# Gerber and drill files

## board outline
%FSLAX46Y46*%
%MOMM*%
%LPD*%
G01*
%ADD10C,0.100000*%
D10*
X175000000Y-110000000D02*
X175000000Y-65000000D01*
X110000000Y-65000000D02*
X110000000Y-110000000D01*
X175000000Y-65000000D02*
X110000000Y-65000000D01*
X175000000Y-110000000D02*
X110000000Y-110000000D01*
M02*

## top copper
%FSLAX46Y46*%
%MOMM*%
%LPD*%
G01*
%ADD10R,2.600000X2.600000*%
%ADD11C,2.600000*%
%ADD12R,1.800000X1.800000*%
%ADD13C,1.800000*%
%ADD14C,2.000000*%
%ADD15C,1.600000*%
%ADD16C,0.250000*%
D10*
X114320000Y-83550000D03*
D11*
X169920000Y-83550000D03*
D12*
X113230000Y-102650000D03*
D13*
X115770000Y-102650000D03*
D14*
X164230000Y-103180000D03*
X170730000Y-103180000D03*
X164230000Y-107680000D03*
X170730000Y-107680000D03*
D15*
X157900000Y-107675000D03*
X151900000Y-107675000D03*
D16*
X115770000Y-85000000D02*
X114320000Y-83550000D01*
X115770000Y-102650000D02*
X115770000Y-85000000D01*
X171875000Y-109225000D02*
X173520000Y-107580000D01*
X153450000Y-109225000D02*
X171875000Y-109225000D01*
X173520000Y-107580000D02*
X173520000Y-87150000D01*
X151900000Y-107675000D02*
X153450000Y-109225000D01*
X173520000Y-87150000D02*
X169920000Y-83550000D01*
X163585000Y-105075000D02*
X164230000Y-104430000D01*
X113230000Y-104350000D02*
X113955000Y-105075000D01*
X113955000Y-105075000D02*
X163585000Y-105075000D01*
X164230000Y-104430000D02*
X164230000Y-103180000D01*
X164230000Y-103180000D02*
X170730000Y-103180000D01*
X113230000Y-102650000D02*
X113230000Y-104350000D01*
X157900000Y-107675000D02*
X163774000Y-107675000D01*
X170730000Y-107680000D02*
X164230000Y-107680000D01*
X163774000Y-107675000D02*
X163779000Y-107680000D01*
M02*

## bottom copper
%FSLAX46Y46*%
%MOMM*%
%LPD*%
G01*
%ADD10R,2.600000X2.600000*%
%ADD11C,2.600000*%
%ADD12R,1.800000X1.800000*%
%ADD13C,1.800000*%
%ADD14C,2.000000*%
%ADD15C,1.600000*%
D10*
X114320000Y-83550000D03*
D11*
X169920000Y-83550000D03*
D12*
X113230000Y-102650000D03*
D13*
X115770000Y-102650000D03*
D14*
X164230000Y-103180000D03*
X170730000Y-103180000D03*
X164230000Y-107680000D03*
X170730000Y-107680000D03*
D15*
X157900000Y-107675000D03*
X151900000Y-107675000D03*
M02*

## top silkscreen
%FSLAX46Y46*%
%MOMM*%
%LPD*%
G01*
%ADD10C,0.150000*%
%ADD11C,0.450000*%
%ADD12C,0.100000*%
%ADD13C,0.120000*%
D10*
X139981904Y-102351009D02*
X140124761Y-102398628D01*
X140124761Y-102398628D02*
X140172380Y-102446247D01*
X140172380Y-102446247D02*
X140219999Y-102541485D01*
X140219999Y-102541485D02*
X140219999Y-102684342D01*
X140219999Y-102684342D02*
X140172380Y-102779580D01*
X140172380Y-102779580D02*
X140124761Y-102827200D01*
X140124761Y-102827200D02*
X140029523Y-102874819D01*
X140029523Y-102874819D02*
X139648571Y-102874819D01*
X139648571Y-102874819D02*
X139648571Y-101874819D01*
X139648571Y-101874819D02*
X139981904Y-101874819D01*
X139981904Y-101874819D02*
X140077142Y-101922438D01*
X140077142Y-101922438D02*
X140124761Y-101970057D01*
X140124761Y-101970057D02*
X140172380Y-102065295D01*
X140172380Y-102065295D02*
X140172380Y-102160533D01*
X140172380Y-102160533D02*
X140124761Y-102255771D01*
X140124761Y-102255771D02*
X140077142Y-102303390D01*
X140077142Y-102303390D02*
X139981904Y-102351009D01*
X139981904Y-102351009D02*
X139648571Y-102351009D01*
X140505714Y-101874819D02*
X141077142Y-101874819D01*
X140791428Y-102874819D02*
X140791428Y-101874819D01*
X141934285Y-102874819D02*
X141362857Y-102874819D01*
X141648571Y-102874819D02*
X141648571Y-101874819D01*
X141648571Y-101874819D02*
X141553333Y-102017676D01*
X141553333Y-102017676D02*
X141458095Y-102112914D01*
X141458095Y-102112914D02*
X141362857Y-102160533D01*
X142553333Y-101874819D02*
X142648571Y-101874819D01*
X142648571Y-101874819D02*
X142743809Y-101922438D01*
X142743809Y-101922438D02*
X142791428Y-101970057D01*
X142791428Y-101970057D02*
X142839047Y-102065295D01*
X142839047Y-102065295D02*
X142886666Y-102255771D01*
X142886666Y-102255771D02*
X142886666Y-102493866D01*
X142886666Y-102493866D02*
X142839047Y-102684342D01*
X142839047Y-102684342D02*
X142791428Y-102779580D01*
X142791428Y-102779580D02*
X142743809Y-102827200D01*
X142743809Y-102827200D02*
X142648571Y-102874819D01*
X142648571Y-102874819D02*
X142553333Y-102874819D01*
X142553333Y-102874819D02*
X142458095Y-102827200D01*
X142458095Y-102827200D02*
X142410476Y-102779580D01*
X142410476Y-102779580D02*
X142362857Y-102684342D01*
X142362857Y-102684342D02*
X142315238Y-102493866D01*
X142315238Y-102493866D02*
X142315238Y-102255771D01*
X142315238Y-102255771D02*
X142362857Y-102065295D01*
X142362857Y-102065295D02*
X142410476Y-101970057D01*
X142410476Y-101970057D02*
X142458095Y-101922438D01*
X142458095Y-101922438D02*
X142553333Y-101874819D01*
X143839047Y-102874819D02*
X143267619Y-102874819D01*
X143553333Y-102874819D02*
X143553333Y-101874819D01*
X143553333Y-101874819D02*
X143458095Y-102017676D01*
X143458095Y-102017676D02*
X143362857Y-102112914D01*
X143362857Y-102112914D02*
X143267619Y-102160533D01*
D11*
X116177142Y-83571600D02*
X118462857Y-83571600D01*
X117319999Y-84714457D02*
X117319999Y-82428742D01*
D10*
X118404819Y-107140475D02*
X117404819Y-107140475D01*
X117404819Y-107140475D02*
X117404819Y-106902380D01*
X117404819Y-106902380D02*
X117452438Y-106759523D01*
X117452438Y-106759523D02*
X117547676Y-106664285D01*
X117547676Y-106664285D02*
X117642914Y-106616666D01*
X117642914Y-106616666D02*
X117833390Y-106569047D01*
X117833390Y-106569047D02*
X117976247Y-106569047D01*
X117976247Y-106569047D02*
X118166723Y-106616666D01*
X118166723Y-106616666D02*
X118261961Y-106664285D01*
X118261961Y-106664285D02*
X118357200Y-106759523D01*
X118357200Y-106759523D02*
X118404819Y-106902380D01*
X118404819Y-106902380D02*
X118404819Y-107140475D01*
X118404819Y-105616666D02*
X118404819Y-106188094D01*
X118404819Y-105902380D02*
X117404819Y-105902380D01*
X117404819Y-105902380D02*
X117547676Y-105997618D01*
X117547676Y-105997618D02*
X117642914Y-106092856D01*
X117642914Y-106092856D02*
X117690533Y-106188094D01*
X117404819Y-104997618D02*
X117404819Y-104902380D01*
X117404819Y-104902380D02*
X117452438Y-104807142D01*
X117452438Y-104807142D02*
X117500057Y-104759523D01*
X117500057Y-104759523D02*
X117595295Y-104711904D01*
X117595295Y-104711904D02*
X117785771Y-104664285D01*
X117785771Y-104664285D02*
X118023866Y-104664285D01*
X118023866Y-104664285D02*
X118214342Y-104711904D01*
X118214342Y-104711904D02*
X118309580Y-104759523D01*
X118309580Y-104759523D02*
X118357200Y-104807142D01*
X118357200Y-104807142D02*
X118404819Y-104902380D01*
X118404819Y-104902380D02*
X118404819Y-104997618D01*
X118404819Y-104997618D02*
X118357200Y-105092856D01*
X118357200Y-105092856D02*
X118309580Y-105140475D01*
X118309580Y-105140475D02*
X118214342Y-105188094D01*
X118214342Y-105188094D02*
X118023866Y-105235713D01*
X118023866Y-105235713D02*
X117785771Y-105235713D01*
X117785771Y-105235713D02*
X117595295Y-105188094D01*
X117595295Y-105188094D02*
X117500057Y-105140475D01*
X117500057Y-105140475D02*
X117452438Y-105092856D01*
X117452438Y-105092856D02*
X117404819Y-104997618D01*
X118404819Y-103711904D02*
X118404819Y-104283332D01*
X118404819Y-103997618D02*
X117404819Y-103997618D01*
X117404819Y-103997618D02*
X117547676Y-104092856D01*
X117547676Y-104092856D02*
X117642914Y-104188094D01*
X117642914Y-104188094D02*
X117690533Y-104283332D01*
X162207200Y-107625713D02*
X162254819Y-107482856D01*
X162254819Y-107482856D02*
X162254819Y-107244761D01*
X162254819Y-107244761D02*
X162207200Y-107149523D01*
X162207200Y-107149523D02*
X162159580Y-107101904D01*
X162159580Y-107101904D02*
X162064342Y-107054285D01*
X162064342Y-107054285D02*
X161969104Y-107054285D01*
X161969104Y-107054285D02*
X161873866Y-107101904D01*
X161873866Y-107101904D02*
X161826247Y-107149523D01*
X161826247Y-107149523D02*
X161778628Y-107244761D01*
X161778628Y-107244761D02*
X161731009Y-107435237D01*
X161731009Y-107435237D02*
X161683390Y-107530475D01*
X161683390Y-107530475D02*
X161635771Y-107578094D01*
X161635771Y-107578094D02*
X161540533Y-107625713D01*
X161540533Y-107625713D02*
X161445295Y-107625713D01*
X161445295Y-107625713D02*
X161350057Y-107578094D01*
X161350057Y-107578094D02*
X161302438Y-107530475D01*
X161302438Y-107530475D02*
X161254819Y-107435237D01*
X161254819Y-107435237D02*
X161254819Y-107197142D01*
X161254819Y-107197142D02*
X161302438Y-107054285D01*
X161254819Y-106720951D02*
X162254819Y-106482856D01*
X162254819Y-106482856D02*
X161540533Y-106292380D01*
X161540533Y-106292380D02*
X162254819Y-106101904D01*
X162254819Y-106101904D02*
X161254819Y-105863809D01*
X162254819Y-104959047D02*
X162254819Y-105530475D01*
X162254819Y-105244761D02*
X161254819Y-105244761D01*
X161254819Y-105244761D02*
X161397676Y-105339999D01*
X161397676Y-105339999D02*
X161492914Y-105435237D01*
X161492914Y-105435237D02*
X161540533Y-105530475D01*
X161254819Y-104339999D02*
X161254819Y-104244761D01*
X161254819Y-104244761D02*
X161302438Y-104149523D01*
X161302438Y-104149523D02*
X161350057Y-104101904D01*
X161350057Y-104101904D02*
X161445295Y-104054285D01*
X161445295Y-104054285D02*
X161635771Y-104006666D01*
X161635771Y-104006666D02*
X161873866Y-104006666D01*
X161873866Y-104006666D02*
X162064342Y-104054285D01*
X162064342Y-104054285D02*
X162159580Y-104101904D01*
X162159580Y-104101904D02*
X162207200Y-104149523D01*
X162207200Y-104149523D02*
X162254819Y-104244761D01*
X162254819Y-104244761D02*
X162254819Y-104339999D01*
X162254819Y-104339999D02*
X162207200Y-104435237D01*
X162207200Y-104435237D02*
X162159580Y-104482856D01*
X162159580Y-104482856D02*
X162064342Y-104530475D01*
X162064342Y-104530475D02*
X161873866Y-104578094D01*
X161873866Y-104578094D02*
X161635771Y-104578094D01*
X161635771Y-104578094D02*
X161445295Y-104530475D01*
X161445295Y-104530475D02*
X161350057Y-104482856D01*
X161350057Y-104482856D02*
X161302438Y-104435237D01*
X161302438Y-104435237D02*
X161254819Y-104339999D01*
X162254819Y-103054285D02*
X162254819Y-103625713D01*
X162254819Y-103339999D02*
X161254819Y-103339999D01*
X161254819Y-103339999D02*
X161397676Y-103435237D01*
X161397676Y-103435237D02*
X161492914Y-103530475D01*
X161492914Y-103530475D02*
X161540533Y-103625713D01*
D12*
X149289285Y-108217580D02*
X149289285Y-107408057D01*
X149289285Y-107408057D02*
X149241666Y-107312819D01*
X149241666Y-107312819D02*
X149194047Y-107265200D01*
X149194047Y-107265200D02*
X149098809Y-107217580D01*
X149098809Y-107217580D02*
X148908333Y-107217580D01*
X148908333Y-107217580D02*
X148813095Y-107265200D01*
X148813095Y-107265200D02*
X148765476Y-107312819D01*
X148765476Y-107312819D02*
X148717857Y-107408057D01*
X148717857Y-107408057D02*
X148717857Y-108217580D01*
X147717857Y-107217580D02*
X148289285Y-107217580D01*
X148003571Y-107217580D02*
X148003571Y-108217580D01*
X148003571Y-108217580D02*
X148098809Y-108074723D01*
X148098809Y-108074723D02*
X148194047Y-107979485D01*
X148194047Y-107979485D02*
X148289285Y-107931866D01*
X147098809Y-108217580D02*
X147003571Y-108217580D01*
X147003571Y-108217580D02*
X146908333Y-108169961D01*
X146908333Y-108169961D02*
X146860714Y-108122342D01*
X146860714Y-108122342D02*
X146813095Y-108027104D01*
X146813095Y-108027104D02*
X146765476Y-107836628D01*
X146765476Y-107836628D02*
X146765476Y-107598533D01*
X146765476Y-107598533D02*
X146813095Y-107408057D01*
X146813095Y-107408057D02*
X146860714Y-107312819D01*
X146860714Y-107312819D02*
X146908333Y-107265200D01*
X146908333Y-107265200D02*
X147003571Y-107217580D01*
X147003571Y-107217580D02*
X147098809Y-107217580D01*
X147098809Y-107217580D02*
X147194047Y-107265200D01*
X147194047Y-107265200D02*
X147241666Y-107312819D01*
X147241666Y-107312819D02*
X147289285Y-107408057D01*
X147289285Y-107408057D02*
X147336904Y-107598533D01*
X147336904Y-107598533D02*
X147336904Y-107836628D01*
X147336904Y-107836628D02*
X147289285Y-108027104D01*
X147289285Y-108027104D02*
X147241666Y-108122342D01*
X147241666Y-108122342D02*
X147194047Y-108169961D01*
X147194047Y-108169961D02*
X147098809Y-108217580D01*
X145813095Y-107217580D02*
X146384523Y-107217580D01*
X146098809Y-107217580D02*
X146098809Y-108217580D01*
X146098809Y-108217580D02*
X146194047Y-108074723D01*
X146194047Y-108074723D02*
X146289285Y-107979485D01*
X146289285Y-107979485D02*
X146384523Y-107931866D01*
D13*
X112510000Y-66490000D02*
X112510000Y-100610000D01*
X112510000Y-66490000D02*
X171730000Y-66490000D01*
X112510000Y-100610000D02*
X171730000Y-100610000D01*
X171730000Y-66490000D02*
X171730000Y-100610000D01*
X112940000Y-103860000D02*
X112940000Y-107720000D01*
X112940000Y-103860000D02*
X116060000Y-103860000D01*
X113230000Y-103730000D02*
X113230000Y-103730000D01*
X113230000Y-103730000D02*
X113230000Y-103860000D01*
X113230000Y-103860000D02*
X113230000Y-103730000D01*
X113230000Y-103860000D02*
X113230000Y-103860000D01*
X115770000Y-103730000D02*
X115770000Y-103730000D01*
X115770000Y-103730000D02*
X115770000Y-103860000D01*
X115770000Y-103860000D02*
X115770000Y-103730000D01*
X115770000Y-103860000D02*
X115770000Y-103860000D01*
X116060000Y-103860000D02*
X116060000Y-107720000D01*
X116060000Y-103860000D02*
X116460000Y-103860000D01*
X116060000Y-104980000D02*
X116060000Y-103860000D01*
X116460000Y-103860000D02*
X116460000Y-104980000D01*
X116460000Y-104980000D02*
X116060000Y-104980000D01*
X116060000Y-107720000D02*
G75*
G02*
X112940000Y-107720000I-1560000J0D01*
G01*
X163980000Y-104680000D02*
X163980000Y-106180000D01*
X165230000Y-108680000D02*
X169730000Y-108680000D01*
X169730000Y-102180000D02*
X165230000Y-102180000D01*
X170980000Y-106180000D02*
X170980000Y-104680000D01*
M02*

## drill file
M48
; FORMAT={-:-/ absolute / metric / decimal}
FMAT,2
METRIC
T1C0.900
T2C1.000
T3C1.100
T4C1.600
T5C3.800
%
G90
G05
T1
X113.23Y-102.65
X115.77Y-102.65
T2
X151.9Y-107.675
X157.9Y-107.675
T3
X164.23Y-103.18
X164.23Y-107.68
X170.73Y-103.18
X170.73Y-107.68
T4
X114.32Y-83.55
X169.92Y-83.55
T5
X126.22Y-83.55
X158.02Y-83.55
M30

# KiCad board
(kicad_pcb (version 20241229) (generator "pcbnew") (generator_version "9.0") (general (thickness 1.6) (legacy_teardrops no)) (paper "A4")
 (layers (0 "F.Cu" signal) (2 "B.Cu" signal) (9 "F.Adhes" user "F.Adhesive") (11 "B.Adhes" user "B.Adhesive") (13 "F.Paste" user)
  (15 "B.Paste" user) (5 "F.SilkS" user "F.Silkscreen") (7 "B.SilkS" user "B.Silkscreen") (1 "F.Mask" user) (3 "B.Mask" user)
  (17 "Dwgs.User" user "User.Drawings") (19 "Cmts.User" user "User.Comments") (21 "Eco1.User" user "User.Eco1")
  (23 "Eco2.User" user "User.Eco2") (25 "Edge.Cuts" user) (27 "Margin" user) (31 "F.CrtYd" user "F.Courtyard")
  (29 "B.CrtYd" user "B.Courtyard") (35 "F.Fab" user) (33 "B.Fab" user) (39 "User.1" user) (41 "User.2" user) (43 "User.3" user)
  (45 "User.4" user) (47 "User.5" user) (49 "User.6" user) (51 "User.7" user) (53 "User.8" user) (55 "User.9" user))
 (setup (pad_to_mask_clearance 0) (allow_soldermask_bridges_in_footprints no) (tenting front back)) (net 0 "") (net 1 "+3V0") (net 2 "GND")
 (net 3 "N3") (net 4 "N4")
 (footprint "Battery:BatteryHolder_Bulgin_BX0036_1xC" (layer "F.Cu") (at 114.32 83.55)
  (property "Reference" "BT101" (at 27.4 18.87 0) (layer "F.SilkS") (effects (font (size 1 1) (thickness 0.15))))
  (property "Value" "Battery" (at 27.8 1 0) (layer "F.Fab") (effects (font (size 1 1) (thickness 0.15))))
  (fp_line (start -1.81 -17.06) (end -1.81 17.06) (stroke (width 0.12) (type solid)) (layer "F.SilkS"))
  (fp_line (start -1.81 -17.06) (end 57.41 -17.06) (stroke (width 0.12) (type solid)) (layer "F.SilkS"))
  (fp_line (start -1.81 17.06) (end 57.41 17.06) (stroke (width 0.12) (type solid)) (layer "F.SilkS"))
  (fp_line (start 57.41 -17.06) (end 57.41 17.06) (stroke (width 0.12) (type solid)) (layer "F.SilkS"))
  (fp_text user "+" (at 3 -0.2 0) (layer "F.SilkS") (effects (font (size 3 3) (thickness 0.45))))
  (pad "" np_thru_hole circle (at 11.9 0) (size 3.8 3.8) (drill 3.8) (layers "*.Cu" "*.Mask"))
  (pad "" np_thru_hole circle (at 43.7 0) (size 3.8 3.8) (drill 3.8) (layers "*.Cu" "*.Mask"))
  (pad "1" thru_hole rect (at 0 0) (size 2.6 2.6) (drill 1.6) (layers "*.Cu" "*.Mask") (remove_unused_layers no) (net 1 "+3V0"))
  (pad "2" thru_hole circle (at 55.6 0) (size 2.6 2.6) (drill 1.6) (layers "*.Cu" "*.Mask") (remove_unused_layers no) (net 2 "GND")))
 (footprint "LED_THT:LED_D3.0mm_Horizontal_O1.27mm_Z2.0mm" (layer "F.Cu") (at 113.23 102.65)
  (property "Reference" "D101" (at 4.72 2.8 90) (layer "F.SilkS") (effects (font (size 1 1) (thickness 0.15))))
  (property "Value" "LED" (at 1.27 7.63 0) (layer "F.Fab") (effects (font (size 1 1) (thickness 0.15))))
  (fp_line (start -0.29 1.21) (end -0.29 5.07) (stroke (width 0.12) (type solid)) (layer "F.SilkS"))
  (fp_line (start -0.29 1.21) (end 2.83 1.21) (stroke (width 0.12) (type solid)) (layer "F.SilkS"))
  (fp_line (start 0 1.08) (end 0 1.08) (stroke (width 0.12) (type solid)) (layer "F.SilkS"))
  (fp_line (start 0 1.08) (end 0 1.21) (stroke (width 0.12) (type solid)) (layer "F.SilkS"))
  (fp_line (start 0 1.21) (end 0 1.08) (stroke (width 0.12) (type solid)) (layer "F.SilkS"))
  (fp_line (start 0 1.21) (end 0 1.21) (stroke (width 0.12) (type solid)) (layer "F.SilkS"))
  (fp_line (start 2.54 1.08) (end 2.54 1.08) (stroke (width 0.12) (type solid)) (layer "F.SilkS"))
  (fp_line (start 2.54 1.08) (end 2.54 1.21) (stroke (width 0.12) (type solid)) (layer "F.SilkS"))
  (fp_line (start 2.54 1.21) (end 2.54 1.08) (stroke (width 0.12) (type solid)) (layer "F.SilkS"))
  (fp_line (start 2.54 1.21) (end 2.54 1.21) (stroke (width 0.12) (type solid)) (layer "F.SilkS"))
  (fp_line (start 2.83 1.21) (end 2.83 5.07) (stroke (width 0.12) (type solid)) (layer "F.SilkS"))
  (fp_line (start 2.83 1.21) (end 3.23 1.21) (stroke (width 0.12) (type solid)) (layer "F.SilkS"))
  (fp_line (start 2.83 2.33) (end 2.83 1.21) (stroke (width 0.12) (type solid)) (layer "F.SilkS"))
  (fp_line (start 3.23 1.21) (end 3.23 2.33) (stroke (width 0.12) (type solid)) (layer "F.SilkS"))
  (fp_line (start 3.23 2.33) (end 2.83 2.33) (stroke (width 0.12) (type solid)) (layer "F.SilkS"))
  (fp_arc (start 2.83 5.07) (mid 1.27 6.63) (end -0.29 5.07) (stroke (width 0.12) (type solid)) (layer "F.SilkS"))
  (pad "1" thru_hole rect (at 0 0) (size 1.8 1.8) (drill 0.9) (layers "*.Cu" "*.Mask") (remove_unused_layers no) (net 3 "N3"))
  (pad "2" thru_hole circle (at 2.54 0) (size 1.8 1.8) (drill 0.9) (layers "*.Cu" "*.Mask") (remove_unused_layers no) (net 1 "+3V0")))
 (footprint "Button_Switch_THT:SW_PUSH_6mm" (layer "F.Cu") (at 164.23 103.18)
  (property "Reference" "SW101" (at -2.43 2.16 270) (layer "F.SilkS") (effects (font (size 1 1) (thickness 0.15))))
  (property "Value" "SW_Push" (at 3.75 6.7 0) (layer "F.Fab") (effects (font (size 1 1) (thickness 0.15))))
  (fp_line (start -0.25 1.5) (end -0.25 3) (stroke (width 0.12) (type solid)) (layer "F.SilkS"))
  (fp_line (start 1 5.5) (end 5.5 5.5) (stroke (width 0.12) (type solid)) (layer "F.SilkS"))
  (fp_line (start 5.5 -1) (end 1 -1) (stroke (width 0.12) (type solid)) (layer "F.SilkS"))
  (fp_line (start 6.75 3) (end 6.75 1.5) (stroke (width 0.12) (type solid)) (layer "F.SilkS"))
  (pad "1" thru_hole circle (at 0 0 90) (size 2 2) (drill 1.1) (layers "*.Cu" "*.Mask") (remove_unused_layers no) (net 3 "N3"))
  (pad "1" thru_hole circle (at 6.5 0 90) (size 2 2) (drill 1.1) (layers "*.Cu" "*.Mask") (remove_unused_layers no) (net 3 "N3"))
  (pad "2" thru_hole circle (at 0 4.5 90) (size 2 2) (drill 1.1) (layers "*.Cu" "*.Mask") (remove_unused_layers no) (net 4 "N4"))
  (pad "2" thru_hole circle (at 6.5 4.5 90) (size 2 2) (drill 1.1) (layers "*.Cu" "*.Mask") (remove_unused_layers no) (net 4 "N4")))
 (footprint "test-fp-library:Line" (layer "F.Cu") (at 154.9 107.675 180)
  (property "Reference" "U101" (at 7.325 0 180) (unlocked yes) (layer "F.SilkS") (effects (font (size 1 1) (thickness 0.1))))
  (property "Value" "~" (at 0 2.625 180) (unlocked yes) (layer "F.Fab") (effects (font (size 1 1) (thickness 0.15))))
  (pad "1" thru_hole circle (at -3 0 180) (size 1.6 1.6) (drill 1) (layers "*.Cu" "*.Mask") (remove_unused_layers no) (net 4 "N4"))
  (pad "2" thru_hole circle (at 3 0 180) (size 1.6 1.6) (drill 1) (layers "*.Cu" "*.Mask") (remove_unused_layers no) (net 2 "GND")))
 (gr_line (start 175 110) (end 175 65) (stroke (width 0.1) (type default)) (layer "Edge.Cuts"))
 (gr_line (start 110 65) (end 110 110) (stroke (width 0.1) (type default)) (layer "Edge.Cuts"))
 (gr_line (start 175 65) (end 110 65) (stroke (width 0.1) (type default)) (layer "Edge.Cuts"))
 (gr_line (start 175 110) (end 110 110) (stroke (width 0.1) (type default)) (layer "Edge.Cuts"))
 (segment (start 115.77 85) (end 114.32 83.55) (width 0.25) (layer "F.Cu") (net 1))
 (segment (start 115.77 102.65) (end 115.77 85) (width 0.25) (layer "F.Cu") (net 1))
 (segment (start 171.875 109.225) (end 173.52 107.58) (width 0.25) (layer "F.Cu") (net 2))
 (segment (start 153.45 109.225) (end 171.875 109.225) (width 0.25) (layer "F.Cu") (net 2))
 (segment (start 173.52 107.58) (end 173.52 87.15) (width 0.25) (layer "F.Cu") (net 2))
 (segment (start 151.9 107.675) (end 153.45 109.225) (width 0.25) (layer "F.Cu") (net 2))
 (segment (start 173.52 87.15) (end 169.92 83.55) (width 0.25) (layer "F.Cu") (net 2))
 (segment (start 163.585 105.075) (end 164.23 104.43) (width 0.25) (layer "F.Cu") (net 3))
 (segment (start 113.23 104.35) (end 113.955 105.075) (width 0.25) (layer "F.Cu") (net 3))
 (segment (start 113.955 105.075) (end 163.585 105.075) (width 0.25) (layer "F.Cu") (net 3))
 (segment (start 164.23 104.43) (end 164.23 103.18) (width 0.25) (layer "F.Cu") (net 3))
 (segment (start 164.23 103.18) (end 170.73 103.18) (width 0.25) (layer "F.Cu") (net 3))
 (segment (start 113.23 102.65) (end 113.23 104.35) (width 0.25) (layer "F.Cu") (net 3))
 (segment (start 157.9 107.675) (end 163.774 107.675) (width 0.25) (layer "F.Cu") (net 4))
 (segment (start 170.73 107.68) (end 164.23 107.68) (width 0.25) (layer "F.Cu") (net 4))
 (segment (start 163.774 107.675) (end 163.779 107.68) (width 0.25) (layer "F.Cu") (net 4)))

